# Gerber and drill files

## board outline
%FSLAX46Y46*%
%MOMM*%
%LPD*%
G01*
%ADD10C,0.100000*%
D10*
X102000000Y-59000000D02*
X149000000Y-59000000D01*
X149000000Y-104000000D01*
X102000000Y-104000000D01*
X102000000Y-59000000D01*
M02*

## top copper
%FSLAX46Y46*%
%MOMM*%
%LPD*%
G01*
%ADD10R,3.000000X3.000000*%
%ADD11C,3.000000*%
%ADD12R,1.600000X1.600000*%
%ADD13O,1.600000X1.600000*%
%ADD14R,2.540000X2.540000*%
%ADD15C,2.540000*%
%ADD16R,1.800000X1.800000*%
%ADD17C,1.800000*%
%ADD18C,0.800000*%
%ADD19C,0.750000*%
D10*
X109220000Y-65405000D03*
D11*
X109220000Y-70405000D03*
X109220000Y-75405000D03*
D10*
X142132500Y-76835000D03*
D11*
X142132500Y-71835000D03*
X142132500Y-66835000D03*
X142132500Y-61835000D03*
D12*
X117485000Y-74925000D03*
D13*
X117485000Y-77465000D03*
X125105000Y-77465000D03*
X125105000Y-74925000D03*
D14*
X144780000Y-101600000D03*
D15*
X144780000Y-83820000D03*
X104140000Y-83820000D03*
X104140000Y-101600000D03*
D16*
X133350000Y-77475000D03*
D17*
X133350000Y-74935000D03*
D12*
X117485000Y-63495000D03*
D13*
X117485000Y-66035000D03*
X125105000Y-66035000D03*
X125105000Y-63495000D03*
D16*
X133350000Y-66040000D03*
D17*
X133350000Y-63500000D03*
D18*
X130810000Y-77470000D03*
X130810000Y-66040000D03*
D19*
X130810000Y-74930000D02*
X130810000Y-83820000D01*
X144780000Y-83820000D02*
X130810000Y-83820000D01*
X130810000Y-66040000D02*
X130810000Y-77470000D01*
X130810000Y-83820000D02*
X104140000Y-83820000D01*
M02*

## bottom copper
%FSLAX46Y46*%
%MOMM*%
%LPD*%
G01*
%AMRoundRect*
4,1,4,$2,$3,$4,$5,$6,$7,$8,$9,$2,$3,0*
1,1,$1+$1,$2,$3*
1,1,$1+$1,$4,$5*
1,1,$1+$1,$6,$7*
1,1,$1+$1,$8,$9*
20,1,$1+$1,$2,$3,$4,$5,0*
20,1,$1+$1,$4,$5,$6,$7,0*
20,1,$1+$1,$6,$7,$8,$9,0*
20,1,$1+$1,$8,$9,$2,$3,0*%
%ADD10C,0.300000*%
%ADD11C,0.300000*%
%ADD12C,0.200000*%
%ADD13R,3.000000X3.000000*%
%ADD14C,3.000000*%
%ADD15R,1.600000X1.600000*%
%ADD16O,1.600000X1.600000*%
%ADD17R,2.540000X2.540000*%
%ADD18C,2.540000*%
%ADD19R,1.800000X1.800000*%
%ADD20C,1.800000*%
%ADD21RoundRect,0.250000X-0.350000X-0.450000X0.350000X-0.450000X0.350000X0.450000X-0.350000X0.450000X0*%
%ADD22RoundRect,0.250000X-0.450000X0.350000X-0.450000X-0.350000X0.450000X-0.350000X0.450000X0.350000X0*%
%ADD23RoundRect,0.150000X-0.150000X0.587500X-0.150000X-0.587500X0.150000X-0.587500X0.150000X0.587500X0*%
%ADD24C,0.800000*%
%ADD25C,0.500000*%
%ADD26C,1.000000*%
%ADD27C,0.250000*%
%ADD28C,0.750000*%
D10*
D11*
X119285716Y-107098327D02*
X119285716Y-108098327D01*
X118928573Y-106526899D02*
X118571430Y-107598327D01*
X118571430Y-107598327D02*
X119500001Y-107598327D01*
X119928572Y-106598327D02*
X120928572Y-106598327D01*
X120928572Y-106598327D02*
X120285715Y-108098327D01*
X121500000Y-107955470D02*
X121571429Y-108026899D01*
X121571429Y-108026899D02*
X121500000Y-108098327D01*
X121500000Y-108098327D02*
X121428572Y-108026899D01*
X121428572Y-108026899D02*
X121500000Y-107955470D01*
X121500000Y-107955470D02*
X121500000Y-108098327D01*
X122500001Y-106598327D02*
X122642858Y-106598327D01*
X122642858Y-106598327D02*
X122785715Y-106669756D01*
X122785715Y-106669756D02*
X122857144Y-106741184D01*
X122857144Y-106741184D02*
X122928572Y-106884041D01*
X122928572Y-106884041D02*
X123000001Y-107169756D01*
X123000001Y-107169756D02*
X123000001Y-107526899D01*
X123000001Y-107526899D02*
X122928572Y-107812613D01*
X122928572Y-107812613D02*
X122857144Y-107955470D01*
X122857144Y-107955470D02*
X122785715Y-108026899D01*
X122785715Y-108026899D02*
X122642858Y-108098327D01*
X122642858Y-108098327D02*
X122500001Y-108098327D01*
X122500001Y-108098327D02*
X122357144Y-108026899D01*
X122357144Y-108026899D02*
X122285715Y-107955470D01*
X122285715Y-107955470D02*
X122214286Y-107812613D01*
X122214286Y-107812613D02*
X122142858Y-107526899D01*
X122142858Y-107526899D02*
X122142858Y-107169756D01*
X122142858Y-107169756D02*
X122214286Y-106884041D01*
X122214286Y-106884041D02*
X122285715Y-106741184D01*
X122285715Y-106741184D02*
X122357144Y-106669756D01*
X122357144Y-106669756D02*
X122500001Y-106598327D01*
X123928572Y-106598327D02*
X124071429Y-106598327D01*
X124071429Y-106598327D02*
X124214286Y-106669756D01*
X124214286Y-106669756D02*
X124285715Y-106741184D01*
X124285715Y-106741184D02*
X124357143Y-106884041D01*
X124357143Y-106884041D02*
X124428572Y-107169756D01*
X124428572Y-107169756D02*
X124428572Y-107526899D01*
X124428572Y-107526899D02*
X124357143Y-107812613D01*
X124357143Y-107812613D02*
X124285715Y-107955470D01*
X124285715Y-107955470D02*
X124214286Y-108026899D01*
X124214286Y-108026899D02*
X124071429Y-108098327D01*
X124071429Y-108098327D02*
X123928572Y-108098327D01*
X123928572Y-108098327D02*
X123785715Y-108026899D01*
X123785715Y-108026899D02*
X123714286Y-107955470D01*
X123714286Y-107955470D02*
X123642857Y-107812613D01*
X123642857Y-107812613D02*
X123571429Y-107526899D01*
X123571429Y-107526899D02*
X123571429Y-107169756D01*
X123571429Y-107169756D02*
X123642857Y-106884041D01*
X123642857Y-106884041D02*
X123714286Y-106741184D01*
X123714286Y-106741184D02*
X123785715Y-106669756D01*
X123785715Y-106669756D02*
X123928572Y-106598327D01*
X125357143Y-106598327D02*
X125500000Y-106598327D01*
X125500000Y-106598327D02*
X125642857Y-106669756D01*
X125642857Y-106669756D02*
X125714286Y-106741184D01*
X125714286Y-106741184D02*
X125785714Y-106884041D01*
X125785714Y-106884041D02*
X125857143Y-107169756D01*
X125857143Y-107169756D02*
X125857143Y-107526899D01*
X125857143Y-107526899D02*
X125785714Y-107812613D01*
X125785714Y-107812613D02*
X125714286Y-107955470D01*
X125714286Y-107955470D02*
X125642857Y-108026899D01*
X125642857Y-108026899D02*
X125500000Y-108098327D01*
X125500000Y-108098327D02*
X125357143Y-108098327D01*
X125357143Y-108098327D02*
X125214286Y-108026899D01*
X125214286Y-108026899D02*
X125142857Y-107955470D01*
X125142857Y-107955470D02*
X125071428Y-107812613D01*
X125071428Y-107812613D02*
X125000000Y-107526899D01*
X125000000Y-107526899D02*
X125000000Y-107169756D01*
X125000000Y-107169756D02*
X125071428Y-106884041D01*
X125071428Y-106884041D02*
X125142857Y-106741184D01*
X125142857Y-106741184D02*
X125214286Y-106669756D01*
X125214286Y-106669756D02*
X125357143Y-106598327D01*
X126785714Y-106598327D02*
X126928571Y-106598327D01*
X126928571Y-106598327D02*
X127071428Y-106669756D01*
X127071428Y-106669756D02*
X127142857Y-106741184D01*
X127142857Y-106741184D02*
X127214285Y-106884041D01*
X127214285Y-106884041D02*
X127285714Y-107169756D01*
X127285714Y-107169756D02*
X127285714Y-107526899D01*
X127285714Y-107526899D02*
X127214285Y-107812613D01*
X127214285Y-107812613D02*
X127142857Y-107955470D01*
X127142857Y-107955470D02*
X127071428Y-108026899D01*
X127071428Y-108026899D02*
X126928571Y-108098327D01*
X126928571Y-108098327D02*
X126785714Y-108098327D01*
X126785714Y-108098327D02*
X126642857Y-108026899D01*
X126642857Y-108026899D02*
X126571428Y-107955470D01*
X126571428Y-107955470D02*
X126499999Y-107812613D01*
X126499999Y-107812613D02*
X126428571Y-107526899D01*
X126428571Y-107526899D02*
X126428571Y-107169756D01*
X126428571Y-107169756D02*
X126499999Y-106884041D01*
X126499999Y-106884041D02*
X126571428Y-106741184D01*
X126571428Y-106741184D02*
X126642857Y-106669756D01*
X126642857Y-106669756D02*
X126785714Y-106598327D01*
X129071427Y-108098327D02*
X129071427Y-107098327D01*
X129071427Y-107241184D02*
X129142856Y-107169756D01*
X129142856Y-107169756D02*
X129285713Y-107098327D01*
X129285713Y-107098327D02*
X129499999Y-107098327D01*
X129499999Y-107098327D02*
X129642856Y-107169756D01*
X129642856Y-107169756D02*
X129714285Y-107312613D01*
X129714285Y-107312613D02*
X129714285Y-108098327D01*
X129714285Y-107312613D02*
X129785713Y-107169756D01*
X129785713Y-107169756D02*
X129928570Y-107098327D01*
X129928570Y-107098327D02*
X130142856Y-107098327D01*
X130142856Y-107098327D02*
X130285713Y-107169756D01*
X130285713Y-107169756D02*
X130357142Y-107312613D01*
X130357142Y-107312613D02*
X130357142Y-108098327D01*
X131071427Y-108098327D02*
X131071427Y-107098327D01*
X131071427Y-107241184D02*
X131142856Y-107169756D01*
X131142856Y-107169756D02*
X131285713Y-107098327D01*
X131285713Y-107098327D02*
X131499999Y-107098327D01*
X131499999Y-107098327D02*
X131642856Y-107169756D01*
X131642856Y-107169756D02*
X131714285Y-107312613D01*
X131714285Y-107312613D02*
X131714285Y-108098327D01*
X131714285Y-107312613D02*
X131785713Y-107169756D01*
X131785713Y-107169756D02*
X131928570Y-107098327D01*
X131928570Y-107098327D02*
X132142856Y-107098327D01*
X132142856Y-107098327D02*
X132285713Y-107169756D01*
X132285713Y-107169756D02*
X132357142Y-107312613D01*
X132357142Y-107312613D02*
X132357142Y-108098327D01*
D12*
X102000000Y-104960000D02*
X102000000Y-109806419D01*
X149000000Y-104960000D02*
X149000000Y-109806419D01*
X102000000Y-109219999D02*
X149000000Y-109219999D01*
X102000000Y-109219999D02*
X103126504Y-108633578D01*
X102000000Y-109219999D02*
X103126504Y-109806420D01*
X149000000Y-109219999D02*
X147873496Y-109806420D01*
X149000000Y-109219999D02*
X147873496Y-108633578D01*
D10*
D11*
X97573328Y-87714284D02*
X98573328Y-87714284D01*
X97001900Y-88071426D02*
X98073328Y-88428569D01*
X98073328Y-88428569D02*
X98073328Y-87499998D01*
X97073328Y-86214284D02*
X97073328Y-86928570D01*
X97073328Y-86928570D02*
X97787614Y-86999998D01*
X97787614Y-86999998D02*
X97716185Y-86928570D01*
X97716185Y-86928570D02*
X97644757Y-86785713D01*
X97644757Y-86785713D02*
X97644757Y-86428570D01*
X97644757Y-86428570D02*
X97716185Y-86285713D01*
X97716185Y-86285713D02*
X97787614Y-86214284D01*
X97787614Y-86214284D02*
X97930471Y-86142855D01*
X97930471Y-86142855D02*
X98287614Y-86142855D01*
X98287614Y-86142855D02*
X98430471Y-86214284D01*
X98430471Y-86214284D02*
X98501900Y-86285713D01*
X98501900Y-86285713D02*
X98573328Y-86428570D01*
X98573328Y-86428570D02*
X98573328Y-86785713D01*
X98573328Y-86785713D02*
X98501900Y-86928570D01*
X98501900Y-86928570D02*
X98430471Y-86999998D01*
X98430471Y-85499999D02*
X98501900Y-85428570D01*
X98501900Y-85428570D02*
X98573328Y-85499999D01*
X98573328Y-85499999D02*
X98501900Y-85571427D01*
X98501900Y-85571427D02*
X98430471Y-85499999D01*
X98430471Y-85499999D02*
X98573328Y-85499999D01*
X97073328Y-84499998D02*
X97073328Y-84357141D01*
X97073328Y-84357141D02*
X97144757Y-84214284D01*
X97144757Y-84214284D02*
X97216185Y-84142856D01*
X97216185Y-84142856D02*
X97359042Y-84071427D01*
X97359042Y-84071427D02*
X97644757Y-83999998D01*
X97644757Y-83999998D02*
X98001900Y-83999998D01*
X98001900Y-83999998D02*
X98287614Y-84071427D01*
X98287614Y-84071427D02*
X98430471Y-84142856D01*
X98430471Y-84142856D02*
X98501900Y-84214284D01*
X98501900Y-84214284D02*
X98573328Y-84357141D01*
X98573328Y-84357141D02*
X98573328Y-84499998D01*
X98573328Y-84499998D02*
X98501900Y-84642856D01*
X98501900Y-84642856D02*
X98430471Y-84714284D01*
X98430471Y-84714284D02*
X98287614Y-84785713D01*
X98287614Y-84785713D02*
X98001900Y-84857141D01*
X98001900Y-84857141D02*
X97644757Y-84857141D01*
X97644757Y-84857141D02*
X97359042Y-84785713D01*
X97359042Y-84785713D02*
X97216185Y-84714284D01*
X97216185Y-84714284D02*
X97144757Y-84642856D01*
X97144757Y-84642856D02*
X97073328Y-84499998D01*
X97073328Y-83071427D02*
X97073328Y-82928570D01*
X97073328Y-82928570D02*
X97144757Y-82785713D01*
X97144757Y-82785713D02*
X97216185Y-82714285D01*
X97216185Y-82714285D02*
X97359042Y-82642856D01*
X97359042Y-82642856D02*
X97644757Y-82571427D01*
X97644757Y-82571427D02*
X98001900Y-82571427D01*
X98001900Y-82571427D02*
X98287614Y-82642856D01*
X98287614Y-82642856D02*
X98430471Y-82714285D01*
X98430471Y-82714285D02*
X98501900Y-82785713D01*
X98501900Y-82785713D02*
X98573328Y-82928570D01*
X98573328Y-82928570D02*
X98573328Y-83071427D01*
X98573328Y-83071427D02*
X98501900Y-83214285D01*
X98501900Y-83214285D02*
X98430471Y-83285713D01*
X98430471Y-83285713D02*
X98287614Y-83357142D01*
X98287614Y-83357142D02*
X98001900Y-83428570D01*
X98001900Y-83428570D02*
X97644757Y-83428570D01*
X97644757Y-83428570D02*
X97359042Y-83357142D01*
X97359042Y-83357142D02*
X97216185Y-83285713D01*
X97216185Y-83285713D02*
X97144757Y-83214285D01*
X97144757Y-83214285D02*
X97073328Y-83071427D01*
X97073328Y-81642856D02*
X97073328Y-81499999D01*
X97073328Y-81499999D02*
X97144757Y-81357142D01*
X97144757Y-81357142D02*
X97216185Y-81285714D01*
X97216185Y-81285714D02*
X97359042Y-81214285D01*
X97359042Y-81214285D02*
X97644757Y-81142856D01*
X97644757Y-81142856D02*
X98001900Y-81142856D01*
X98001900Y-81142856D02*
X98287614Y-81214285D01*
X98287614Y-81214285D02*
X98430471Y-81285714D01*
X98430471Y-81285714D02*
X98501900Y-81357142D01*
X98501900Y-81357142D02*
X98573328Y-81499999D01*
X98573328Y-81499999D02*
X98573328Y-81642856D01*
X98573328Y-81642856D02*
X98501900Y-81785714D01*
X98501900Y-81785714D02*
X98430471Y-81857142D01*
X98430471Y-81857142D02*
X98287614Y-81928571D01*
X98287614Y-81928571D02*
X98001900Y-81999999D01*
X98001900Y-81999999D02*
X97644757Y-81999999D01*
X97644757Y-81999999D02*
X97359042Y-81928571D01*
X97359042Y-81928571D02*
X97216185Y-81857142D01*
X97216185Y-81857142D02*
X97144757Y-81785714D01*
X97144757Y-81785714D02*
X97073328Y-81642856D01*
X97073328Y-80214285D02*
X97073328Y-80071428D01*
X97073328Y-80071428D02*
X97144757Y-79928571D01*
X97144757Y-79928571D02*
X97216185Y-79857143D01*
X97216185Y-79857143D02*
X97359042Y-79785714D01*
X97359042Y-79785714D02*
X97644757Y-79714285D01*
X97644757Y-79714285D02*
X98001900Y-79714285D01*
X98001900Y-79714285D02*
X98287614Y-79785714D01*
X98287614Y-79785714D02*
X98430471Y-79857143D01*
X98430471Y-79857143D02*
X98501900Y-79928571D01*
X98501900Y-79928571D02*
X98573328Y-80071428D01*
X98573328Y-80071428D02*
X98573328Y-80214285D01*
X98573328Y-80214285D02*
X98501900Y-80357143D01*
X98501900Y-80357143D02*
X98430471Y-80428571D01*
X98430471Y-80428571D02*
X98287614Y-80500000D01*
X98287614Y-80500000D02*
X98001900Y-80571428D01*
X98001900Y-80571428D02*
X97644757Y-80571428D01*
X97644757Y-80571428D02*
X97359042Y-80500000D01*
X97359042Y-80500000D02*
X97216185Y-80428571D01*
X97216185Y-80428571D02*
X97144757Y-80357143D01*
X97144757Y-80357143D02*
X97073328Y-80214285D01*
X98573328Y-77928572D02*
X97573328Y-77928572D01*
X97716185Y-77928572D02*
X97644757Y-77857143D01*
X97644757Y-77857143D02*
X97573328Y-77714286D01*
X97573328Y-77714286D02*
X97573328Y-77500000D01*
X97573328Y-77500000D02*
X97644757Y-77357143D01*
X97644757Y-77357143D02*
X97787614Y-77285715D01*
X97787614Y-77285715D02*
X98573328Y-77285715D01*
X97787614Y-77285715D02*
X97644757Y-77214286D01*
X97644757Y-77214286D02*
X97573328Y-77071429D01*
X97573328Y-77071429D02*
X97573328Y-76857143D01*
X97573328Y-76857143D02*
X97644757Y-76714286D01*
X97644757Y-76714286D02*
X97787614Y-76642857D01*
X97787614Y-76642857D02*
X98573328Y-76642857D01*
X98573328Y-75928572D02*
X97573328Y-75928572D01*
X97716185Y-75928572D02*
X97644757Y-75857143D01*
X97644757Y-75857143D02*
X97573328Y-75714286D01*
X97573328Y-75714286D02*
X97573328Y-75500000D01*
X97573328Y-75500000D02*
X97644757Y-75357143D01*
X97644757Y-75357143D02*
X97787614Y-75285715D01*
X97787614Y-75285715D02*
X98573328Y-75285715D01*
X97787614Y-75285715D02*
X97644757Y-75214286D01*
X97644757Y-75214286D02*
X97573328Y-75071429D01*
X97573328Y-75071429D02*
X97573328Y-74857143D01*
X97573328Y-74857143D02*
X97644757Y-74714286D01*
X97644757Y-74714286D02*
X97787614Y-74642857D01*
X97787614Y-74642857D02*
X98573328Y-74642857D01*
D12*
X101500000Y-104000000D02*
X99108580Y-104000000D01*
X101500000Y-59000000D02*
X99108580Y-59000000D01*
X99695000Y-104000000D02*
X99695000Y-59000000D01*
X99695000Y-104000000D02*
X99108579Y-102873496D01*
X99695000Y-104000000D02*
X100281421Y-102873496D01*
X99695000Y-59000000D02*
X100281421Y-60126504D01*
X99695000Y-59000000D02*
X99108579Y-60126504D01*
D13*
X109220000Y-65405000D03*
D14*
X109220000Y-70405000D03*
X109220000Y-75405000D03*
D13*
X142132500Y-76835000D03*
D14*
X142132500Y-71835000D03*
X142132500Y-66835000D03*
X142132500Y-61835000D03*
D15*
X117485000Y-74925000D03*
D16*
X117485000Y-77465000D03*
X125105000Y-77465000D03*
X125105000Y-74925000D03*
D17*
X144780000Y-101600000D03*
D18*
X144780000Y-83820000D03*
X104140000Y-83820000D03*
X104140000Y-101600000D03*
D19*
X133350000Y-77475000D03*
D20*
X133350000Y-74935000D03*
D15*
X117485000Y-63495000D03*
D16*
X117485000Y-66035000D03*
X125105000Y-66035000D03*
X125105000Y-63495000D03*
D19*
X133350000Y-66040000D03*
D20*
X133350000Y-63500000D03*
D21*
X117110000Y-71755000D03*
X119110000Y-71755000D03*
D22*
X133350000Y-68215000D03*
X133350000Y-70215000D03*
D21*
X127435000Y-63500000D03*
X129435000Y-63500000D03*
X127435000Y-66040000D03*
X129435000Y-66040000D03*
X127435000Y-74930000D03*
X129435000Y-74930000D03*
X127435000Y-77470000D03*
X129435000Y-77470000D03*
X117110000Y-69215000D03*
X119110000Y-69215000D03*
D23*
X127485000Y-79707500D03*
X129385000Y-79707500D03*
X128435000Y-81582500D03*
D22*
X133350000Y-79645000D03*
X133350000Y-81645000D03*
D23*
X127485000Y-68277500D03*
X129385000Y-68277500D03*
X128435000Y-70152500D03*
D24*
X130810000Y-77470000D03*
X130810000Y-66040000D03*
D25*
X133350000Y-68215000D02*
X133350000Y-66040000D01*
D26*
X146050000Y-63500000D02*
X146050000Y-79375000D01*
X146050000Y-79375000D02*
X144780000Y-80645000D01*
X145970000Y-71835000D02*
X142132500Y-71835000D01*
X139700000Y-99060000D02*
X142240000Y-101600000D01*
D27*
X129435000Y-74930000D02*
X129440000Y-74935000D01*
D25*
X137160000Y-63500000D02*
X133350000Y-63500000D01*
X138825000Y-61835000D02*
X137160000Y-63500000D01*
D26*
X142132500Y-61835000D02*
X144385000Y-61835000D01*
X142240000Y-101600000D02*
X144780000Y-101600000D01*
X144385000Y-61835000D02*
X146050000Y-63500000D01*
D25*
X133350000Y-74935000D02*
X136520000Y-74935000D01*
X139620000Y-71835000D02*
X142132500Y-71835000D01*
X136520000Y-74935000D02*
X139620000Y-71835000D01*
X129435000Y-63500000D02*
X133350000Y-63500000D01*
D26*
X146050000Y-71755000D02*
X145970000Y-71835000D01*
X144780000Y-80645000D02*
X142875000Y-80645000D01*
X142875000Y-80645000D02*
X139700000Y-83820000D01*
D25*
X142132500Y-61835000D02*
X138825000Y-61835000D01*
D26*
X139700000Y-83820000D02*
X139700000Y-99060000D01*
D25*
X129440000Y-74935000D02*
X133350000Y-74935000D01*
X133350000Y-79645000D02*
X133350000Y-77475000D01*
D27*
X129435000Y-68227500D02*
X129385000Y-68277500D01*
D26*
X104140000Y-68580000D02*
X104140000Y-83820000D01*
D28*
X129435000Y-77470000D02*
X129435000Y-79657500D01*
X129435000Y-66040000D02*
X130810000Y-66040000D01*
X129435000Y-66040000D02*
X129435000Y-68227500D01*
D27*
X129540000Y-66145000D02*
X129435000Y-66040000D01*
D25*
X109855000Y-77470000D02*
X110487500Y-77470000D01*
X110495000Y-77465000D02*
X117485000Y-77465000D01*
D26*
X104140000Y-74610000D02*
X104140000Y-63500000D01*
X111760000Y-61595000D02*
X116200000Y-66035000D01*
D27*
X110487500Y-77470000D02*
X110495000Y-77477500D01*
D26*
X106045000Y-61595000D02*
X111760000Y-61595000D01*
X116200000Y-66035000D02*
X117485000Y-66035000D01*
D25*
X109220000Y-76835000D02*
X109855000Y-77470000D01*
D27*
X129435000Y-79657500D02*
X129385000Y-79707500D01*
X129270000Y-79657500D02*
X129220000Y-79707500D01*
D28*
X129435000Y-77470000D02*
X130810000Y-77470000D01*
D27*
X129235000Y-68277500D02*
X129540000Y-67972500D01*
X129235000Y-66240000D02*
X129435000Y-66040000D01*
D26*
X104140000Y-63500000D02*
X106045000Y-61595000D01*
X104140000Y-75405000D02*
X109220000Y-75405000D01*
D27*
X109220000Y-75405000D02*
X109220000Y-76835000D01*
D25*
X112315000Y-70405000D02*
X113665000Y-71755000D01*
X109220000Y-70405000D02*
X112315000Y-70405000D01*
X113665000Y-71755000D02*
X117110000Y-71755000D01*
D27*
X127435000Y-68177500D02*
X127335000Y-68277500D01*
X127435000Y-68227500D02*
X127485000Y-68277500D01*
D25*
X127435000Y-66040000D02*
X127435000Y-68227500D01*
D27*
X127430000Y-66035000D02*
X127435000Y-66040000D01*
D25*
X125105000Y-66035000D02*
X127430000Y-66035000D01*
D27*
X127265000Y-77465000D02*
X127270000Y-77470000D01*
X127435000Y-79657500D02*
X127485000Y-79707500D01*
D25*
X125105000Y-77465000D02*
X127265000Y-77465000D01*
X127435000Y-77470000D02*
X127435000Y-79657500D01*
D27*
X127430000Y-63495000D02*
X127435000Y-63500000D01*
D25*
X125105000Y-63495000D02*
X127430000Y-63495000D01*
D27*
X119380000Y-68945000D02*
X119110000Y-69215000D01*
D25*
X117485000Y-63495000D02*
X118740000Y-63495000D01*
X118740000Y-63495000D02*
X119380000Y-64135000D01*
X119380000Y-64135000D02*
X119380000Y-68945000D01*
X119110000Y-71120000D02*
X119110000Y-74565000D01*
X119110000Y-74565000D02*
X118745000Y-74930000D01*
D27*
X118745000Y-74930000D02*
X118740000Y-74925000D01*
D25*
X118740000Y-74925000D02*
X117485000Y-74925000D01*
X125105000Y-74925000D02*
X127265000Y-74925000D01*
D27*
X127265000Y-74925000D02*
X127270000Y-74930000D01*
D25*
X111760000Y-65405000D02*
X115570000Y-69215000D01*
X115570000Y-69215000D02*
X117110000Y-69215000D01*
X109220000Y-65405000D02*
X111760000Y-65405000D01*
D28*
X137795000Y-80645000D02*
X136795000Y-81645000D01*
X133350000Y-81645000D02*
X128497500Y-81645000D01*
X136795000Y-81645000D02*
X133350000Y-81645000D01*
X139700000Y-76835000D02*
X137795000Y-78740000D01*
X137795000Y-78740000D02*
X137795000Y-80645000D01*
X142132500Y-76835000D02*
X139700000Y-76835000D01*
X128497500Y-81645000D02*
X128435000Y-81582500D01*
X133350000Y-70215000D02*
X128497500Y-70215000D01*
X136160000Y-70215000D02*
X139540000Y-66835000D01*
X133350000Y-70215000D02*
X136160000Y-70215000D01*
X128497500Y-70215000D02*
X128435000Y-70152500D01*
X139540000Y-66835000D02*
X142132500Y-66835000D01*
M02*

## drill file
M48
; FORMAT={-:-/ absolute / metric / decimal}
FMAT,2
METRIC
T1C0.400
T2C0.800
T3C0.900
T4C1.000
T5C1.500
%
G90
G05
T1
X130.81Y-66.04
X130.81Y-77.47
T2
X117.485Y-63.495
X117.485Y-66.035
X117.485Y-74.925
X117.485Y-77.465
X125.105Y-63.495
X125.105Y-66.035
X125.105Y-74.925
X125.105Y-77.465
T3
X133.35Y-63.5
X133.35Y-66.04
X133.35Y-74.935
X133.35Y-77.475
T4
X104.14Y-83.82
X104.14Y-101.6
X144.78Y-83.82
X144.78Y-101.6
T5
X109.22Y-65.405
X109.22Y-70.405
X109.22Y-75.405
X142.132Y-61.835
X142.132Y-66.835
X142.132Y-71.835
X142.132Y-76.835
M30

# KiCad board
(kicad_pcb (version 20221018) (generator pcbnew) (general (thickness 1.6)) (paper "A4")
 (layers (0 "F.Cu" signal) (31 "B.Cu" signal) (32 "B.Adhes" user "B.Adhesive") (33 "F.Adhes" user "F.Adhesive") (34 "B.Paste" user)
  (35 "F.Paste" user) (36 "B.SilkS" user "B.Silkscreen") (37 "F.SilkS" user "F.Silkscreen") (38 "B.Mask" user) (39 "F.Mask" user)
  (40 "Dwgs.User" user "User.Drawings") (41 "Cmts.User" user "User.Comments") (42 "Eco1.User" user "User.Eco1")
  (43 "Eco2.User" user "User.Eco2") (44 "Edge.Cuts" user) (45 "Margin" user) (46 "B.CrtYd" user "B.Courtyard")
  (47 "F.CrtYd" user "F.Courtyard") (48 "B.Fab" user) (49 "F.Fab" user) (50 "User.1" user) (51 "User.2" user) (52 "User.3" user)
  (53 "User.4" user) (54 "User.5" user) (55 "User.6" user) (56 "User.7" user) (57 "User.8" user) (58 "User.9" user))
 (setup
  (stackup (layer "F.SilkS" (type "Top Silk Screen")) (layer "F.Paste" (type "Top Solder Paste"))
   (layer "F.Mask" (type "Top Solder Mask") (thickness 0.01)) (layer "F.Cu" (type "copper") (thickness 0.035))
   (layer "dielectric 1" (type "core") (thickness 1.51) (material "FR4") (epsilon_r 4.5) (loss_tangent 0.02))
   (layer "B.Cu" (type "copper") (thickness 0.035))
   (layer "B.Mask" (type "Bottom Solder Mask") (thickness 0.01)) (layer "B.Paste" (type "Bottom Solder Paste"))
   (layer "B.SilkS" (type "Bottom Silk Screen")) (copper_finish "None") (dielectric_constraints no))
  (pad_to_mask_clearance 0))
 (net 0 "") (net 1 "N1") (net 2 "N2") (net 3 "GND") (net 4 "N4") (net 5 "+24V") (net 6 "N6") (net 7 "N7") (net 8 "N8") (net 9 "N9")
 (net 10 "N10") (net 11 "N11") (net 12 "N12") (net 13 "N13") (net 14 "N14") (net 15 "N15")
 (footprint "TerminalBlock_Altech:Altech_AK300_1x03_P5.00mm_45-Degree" (layer "F.Cu") (at 109.22 65.405 -90)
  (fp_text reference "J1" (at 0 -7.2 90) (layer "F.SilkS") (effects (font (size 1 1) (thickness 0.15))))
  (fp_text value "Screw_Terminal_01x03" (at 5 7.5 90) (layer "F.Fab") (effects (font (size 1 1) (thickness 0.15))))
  (pad "1" thru_hole rect (at 0 0 270) (size 3 3) (drill 1.5) (layers "*.Cu" "*.Mask") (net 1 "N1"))
  (pad "2" thru_hole circle (at 5 0 270) (size 3 3) (drill 1.5) (layers "*.Cu" "*.Mask") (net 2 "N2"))
  (pad "3" thru_hole circle (at 10 0 270) (size 3 3) (drill 1.5) (layers "*.Cu" "*.Mask") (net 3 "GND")))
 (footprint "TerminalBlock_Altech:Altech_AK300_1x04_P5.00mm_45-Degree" (layer "F.Cu") (at 142.1325 76.835 90)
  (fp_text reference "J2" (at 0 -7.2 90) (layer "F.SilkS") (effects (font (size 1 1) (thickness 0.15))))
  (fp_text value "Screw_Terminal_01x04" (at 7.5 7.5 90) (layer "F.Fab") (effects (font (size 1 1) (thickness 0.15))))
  (pad "1" thru_hole rect (at 0 0 90) (size 3 3) (drill 1.5) (layers "*.Cu" "*.Mask") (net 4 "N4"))
  (pad "2" thru_hole circle (at 5 0 90) (size 3 3) (drill 1.5) (layers "*.Cu" "*.Mask") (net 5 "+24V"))
  (pad "3" thru_hole circle (at 10 0 90) (size 3 3) (drill 1.5) (layers "*.Cu" "*.Mask") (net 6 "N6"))
  (pad "4" thru_hole circle (at 15 0 90) (size 3 3) (drill 1.5) (layers "*.Cu" "*.Mask") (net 5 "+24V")))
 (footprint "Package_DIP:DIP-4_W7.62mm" (layer "F.Cu") (at 117.485 74.925)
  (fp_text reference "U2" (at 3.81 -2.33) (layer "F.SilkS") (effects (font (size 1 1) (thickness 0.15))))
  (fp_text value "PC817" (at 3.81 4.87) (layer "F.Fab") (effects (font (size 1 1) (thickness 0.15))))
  (pad "1" thru_hole rect (at 0 0) (size 1.6 1.6) (drill 0.8) (layers "*.Cu" "*.Mask") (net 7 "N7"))
  (pad "2" thru_hole oval (at 0 2.54) (size 1.6 1.6) (drill 0.8) (layers "*.Cu" "*.Mask") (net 3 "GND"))
  (pad "3" thru_hole oval (at 7.62 2.54) (size 1.6 1.6) (drill 0.8) (layers "*.Cu" "*.Mask") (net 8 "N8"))
  (pad "4" thru_hole oval (at 7.62 0) (size 1.6 1.6) (drill 0.8) (layers "*.Cu" "*.Mask") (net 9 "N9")))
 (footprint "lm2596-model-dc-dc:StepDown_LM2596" (layer "F.Cu") (at 144.78 101.6 180)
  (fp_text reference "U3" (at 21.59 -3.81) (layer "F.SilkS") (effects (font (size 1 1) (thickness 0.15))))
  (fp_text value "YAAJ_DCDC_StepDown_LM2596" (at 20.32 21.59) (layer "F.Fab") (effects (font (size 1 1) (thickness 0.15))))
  (pad "1" thru_hole rect (at 0 0 180) (size 2.54 2.54) (drill 1) (layers "*.Cu" "*.Mask") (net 5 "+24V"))
  (pad "2" thru_hole circle (at 0 17.78 180) (size 2.54 2.54) (drill 1) (layers "*.Cu" "*.Mask") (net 3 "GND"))
  (pad "3" thru_hole circle (at 40.64 17.78 180) (size 2.54 2.54) (drill 1) (layers "*.Cu" "*.Mask") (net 3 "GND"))
  (pad "4" thru_hole circle (at 40.64 0 180) (size 2.54 2.54) (drill 1) (layers "*.Cu" "*.Mask") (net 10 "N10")))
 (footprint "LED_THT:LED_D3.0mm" (layer "F.Cu") (at 133.35 77.475 90)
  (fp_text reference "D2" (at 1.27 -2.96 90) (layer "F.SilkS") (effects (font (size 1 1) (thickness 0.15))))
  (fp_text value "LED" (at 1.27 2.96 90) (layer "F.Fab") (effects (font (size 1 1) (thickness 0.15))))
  (pad "1" thru_hole rect (at 0 0 90) (size 1.8 1.8) (drill 0.9) (layers "*.Cu" "*.Mask") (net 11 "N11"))
  (pad "2" thru_hole circle (at 2.54 0 90) (size 1.8 1.8) (drill 0.9) (layers "*.Cu" "*.Mask") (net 5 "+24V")))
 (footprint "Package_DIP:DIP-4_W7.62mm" (layer "F.Cu") (at 117.485 63.495)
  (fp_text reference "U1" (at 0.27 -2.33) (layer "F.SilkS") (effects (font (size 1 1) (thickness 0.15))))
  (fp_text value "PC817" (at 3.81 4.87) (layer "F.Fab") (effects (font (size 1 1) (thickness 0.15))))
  (pad "1" thru_hole rect (at 0 0) (size 1.6 1.6) (drill 0.8) (layers "*.Cu" "*.Mask") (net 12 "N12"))
  (pad "2" thru_hole oval (at 0 2.54) (size 1.6 1.6) (drill 0.8) (layers "*.Cu" "*.Mask") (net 3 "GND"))
  (pad "3" thru_hole oval (at 7.62 2.54) (size 1.6 1.6) (drill 0.8) (layers "*.Cu" "*.Mask") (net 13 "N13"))
  (pad "4" thru_hole oval (at 7.62 0) (size 1.6 1.6) (drill 0.8) (layers "*.Cu" "*.Mask") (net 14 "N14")))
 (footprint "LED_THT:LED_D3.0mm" (layer "F.Cu") (at 133.35 66.04 90)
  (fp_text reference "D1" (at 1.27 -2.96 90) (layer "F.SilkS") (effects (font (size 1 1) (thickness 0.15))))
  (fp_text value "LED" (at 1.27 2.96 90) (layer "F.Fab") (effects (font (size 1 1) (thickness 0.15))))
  (pad "1" thru_hole rect (at 0 0 90) (size 1.8 1.8) (drill 0.9) (layers "*.Cu" "*.Mask") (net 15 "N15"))
  (pad "2" thru_hole circle (at 2.54 0 90) (size 1.8 1.8) (drill 0.9) (layers "*.Cu" "*.Mask") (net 5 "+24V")))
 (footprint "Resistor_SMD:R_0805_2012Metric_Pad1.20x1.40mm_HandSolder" (layer "B.Cu") (at 118.11 71.755)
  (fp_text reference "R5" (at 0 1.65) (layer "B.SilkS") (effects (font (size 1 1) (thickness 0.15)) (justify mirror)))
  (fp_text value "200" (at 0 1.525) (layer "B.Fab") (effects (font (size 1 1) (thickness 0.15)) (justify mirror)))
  (pad "1" smd roundrect (at -1 0) (size 1.2 1.4) (layers "B.Cu" "B.Paste" "B.Mask") (roundrect_rratio 0.208333) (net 2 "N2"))
  (pad "2" smd roundrect (at 1 0) (size 1.2 1.4) (layers "B.Cu" "B.Paste" "B.Mask") (roundrect_rratio 0.208333) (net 7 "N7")))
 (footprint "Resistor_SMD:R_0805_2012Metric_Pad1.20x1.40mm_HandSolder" (layer "B.Cu") (at 133.35 69.215 -90)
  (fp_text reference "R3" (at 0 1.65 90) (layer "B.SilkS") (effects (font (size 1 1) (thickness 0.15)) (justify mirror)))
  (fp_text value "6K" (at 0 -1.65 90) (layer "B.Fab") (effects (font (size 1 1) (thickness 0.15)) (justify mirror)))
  (pad "1" smd roundrect (at -1 0 270) (size 1.2 1.4) (layers "B.Cu" "B.Paste" "B.Mask") (roundrect_rratio 0.208333) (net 15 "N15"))
  (pad "2" smd roundrect (at 1 0 270) (size 1.2 1.4) (layers "B.Cu" "B.Paste" "B.Mask") (roundrect_rratio 0.208333) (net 6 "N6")))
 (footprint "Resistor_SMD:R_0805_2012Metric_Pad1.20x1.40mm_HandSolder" (layer "B.Cu") (at 128.435 63.5)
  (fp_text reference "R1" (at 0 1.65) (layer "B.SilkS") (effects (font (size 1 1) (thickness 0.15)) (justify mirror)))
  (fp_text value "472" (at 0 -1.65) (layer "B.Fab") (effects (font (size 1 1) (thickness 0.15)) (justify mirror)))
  (pad "1" smd roundrect (at -1 0) (size 1.2 1.4) (layers "B.Cu" "B.Paste" "B.Mask") (roundrect_rratio 0.208333) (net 14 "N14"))
  (pad "2" smd roundrect (at 1 0) (size 1.2 1.4) (layers "B.Cu" "B.Paste" "B.Mask") (roundrect_rratio 0.208333) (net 5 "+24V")))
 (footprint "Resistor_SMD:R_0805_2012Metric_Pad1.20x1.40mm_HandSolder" (layer "B.Cu") (at 128.435 66.04)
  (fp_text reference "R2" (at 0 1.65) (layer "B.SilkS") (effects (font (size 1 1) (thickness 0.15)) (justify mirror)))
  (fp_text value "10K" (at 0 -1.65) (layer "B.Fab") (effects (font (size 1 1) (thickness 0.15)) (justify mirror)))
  (pad "1" smd roundrect (at -1 0) (size 1.2 1.4) (layers "B.Cu" "B.Paste" "B.Mask") (roundrect_rratio 0.208333) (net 13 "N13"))
  (pad "2" smd roundrect (at 1 0) (size 1.2 1.4) (layers "B.Cu" "B.Paste" "B.Mask") (roundrect_rratio 0.208333) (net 3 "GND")))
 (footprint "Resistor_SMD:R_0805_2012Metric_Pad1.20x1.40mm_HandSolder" (layer "B.Cu") (at 128.435 74.93)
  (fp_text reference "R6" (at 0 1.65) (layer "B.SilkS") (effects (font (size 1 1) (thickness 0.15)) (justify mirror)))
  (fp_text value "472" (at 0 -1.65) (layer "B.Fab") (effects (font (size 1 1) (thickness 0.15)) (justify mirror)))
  (pad "1" smd roundrect (at -1 0) (size 1.2 1.4) (layers "B.Cu" "B.Paste" "B.Mask") (roundrect_rratio 0.208333) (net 9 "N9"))
  (pad "2" smd roundrect (at 1 0) (size 1.2 1.4) (layers "B.Cu" "B.Paste" "B.Mask") (roundrect_rratio 0.208333) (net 5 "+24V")))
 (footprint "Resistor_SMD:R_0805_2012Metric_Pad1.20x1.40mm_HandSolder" (layer "B.Cu") (at 128.435 77.47)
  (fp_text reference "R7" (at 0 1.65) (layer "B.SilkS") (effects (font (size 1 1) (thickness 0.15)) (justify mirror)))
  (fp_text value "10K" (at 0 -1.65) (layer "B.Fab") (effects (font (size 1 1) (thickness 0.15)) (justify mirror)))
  (pad "1" smd roundrect (at -1 0) (size 1.2 1.4) (layers "B.Cu" "B.Paste" "B.Mask") (roundrect_rratio 0.208333) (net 8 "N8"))
  (pad "2" smd roundrect (at 1 0) (size 1.2 1.4) (layers "B.Cu" "B.Paste" "B.Mask") (roundrect_rratio 0.208333) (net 3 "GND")))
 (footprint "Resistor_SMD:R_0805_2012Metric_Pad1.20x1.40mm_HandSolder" (layer "B.Cu") (at 118.11 69.215)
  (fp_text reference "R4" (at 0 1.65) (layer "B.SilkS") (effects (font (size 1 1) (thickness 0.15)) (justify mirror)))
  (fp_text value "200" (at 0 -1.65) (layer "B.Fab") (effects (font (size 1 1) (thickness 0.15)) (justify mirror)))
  (pad "1" smd roundrect (at -1 0) (size 1.2 1.4) (layers "B.Cu" "B.Paste" "B.Mask") (roundrect_rratio 0.208333) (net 1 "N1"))
  (pad "2" smd roundrect (at 1 0) (size 1.2 1.4) (layers "B.Cu" "B.Paste" "B.Mask") (roundrect_rratio 0.208333) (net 12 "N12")))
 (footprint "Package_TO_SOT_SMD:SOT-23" (layer "B.Cu") (at 128.435 80.645 -90)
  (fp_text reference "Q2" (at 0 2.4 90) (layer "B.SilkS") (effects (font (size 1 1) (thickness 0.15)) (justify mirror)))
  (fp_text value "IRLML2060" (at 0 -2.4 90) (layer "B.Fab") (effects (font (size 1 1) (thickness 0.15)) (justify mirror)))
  (pad "1" smd roundrect (at -0.9375 0.95 270) (size 1.475 0.6) (layers "B.Cu" "B.Paste" "B.Mask") (roundrect_rratio 0.25) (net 8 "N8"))
  (pad "2" smd roundrect (at -0.9375 -0.95 270) (size 1.475 0.6) (layers "B.Cu" "B.Paste" "B.Mask") (roundrect_rratio 0.25) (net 3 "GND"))
  (pad "3" smd roundrect (at 0.9375 0 270) (size 1.475 0.6) (layers "B.Cu" "B.Paste" "B.Mask") (roundrect_rratio 0.25) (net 4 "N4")))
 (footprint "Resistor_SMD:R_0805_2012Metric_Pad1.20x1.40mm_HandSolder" (layer "B.Cu") (at 133.35 80.645 -90)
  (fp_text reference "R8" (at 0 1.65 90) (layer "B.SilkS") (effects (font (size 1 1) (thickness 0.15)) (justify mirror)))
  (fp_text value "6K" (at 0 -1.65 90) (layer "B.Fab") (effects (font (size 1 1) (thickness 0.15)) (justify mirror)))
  (pad "1" smd roundrect (at -1 0 270) (size 1.2 1.4) (layers "B.Cu" "B.Paste" "B.Mask") (roundrect_rratio 0.208333) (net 11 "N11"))
  (pad "2" smd roundrect (at 1 0 270) (size 1.2 1.4) (layers "B.Cu" "B.Paste" "B.Mask") (roundrect_rratio 0.208333) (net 4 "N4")))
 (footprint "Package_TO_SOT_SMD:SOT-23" (layer "B.Cu") (at 128.435 69.215 -90)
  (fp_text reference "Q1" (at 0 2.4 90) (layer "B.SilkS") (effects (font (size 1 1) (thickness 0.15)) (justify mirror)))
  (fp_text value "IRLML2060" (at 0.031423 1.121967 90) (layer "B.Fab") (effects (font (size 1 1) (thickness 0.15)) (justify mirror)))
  (pad "1" smd roundrect (at -0.9375 0.95 270) (size 1.475 0.6) (layers "B.Cu" "B.Paste" "B.Mask") (roundrect_rratio 0.25) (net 13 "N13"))
  (pad "2" smd roundrect (at -0.9375 -0.95 270) (size 1.475 0.6) (layers "B.Cu" "B.Paste" "B.Mask") (roundrect_rratio 0.25) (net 3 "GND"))
  (pad "3" smd roundrect (at 0.9375 0 270) (size 1.475 0.6) (layers "B.Cu" "B.Paste" "B.Mask") (roundrect_rratio 0.25) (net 6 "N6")))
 (gr_rect (start 102 59) (end 149 104) (stroke (width 0.1) (type default)) (fill none) (layer "Edge.Cuts"))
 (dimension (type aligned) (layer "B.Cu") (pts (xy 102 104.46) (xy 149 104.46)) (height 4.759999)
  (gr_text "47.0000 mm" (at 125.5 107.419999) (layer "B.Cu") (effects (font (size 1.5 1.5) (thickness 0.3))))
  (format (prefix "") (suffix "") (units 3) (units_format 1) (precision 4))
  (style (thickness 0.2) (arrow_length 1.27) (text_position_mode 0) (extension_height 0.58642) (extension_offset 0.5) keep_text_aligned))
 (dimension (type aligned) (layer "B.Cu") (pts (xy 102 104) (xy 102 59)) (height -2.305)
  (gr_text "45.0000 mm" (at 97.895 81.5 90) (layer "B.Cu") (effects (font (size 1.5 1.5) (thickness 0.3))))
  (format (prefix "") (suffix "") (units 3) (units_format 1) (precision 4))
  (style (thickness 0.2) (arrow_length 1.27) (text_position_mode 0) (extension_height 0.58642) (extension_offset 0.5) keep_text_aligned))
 (segment (start 133.35 68.215) (end 133.35 66.04) (width 0.5) (layer "B.Cu") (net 15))
 (segment (start 146.05 63.5) (end 146.05 79.375) (width 1) (layer "B.Cu") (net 5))
 (segment (start 146.05 79.375) (end 144.78 80.645) (width 1) (layer "B.Cu") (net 5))
 (segment (start 145.97 71.835) (end 142.1325 71.835) (width 1) (layer "B.Cu") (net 5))
 (segment (start 139.7 99.06) (end 142.24 101.6) (width 1) (layer "B.Cu") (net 5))
 (segment (start 129.435 74.93) (end 129.44 74.935) (width 0.25) (layer "B.Cu") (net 5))
 (segment (start 137.16 63.5) (end 133.35 63.5) (width 0.5) (layer "B.Cu") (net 5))
 (segment (start 138.825 61.835) (end 137.16 63.5) (width 0.5) (layer "B.Cu") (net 5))
 (segment (start 142.1325 61.835) (end 144.385 61.835) (width 1) (layer "B.Cu") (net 5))
 (segment (start 142.24 101.6) (end 144.78 101.6) (width 1) (layer "B.Cu") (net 5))
 (segment (start 144.385 61.835) (end 146.05 63.5) (width 1) (layer "B.Cu") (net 5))
 (segment (start 133.35 74.935) (end 136.52 74.935) (width 0.5) (layer "B.Cu") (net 5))
 (segment (start 139.62 71.835) (end 142.1325 71.835) (width 0.5) (layer "B.Cu") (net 5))
 (segment (start 136.52 74.935) (end 139.62 71.835) (width 0.5) (layer "B.Cu") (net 5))
 (segment (start 129.435 63.5) (end 133.35 63.5) (width 0.5) (layer "B.Cu") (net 5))
 (segment (start 146.05 71.755) (end 145.97 71.835) (width 1) (layer "B.Cu") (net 5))
 (segment (start 144.78 80.645) (end 142.875 80.645) (width 1) (layer "B.Cu") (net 5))
 (segment (start 142.875 80.645) (end 139.7 83.82) (width 1) (layer "B.Cu") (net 5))
 (segment (start 142.1325 61.835) (end 138.825 61.835) (width 0.5) (layer "B.Cu") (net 5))
 (segment (start 139.7 83.82) (end 139.7 99.06) (width 1) (layer "B.Cu") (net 5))
 (segment (start 129.44 74.935) (end 133.35 74.935) (width 0.5) (layer "B.Cu") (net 5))
 (segment (start 133.35 79.645) (end 133.35 77.475) (width 0.5) (layer "B.Cu") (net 11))
 (segment (start 130.81 74.93) (end 130.81 83.82) (width 0.75) (layer "F.Cu") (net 3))
 (segment (start 144.78 83.82) (end 130.81 83.82) (width 0.75) (layer "F.Cu") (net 3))
 (segment (start 130.81 66.04) (end 130.81 77.47) (width 0.75) (layer "F.Cu") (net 3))
 (segment (start 130.81 83.82) (end 104.14 83.82) (width 0.75) (layer "F.Cu") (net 3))
 (via (at 130.81 77.47) (size 0.8) (drill 0.4) (layers "F.Cu" "B.Cu") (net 3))
 (via (at 130.81 66.04) (size 0.8) (drill 0.4) (layers "F.Cu" "B.Cu") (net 3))
 (segment (start 129.435 68.2275) (end 129.385 68.2775) (width 0.25) (layer "B.Cu") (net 3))
 (segment (start 104.14 68.58) (end 104.14 83.82) (width 1) (layer "B.Cu") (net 3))
 (segment (start 129.435 77.47) (end 129.435 79.6575) (width 0.75) (layer "B.Cu") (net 3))
 (segment (start 129.435 66.04) (end 130.81 66.04) (width 0.75) (layer "B.Cu") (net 3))
 (segment (start 129.435 66.04) (end 129.435 68.2275) (width 0.75) (layer "B.Cu") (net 3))
 (segment (start 129.54 66.145) (end 129.435 66.04) (width 0.25) (layer "B.Cu") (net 3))
 (segment (start 109.855 77.47) (end 110.4875 77.47) (width 0.5) (layer "B.Cu") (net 3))
 (segment (start 110.495 77.465) (end 117.485 77.465) (width 0.5) (layer "B.Cu") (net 3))
 (segment (start 104.14 74.61) (end 104.14 63.5) (width 1) (layer "B.Cu") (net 3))
 (segment (start 111.76 61.595) (end 116.2 66.035) (width 1) (layer "B.Cu") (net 3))
 (segment (start 110.4875 77.47) (end 110.495 77.4775) (width 0.25) (layer "B.Cu") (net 3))
 (segment (start 106.045 61.595) (end 111.76 61.595) (width 1) (layer "B.Cu") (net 3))
 (segment (start 116.2 66.035) (end 117.485 66.035) (width 1) (layer "B.Cu") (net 3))
 (segment (start 109.22 76.835) (end 109.855 77.47) (width 0.5) (layer "B.Cu") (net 3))
 (segment (start 129.435 79.6575) (end 129.385 79.7075) (width 0.25) (layer "B.Cu") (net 3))
 (segment (start 129.27 79.6575) (end 129.22 79.7075) (width 0.25) (layer "B.Cu") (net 3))
 (segment (start 129.435 77.47) (end 130.81 77.47) (width 0.75) (layer "B.Cu") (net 3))
 (segment (start 129.235 68.2775) (end 129.54 67.9725) (width 0.25) (layer "B.Cu") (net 3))
 (segment (start 129.235 66.24) (end 129.435 66.04) (width 0.25) (layer "B.Cu") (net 3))
 (segment (start 104.14 63.5) (end 106.045 61.595) (width 1) (layer "B.Cu") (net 3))
 (segment (start 104.14 75.405) (end 109.22 75.405) (width 1) (layer "B.Cu") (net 3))
 (segment (start 109.22 75.405) (end 109.22 76.835) (width 0.25) (layer "B.Cu") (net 3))
 (segment (start 112.315 70.405) (end 113.665 71.755) (width 0.5) (layer "B.Cu") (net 2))
 (segment (start 109.22 70.405) (end 112.315 70.405) (width 0.5) (layer "B.Cu") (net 2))
 (segment (start 113.665 71.755) (end 117.11 71.755) (width 0.5) (layer "B.Cu") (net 2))
 (segment (start 127.435 68.1775) (end 127.335 68.2775) (width 0.25) (layer "B.Cu") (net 13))
 (segment (start 127.435 68.2275) (end 127.485 68.2775) (width 0.25) (layer "B.Cu") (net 13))
 (segment (start 127.435 66.04) (end 127.435 68.2275) (width 0.5) (layer "B.Cu") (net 13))
 (segment (start 127.43 66.035) (end 127.435 66.04) (width 0.25) (layer "B.Cu") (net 13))
 (segment (start 125.105 66.035) (end 127.43 66.035) (width 0.5) (layer "B.Cu") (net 13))
 (segment (start 127.265 77.465) (end 127.27 77.47) (width 0.25) (layer "B.Cu") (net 8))
 (segment (start 127.435 79.6575) (end 127.485 79.7075) (width 0.25) (layer "B.Cu") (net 8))
 (segment (start 125.105 77.465) (end 127.265 77.465) (width 0.5) (layer "B.Cu") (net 8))
 (segment (start 127.435 77.47) (end 127.435 79.6575) (width 0.5) (layer "B.Cu") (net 8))
 (segment (start 127.43 63.495) (end 127.435 63.5) (width 0.25) (layer "B.Cu") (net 14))
 (segment (start 125.105 63.495) (end 127.43 63.495) (width 0.5) (layer "B.Cu") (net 14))
 (segment (start 119.38 68.945) (end 119.11 69.215) (width 0.25) (layer "B.Cu") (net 12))
 (segment (start 117.485 63.495) (end 118.74 63.495) (width 0.5) (layer "B.Cu") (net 12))
 (segment (start 118.74 63.495) (end 119.38 64.135) (width 0.5) (layer "B.Cu") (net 12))
 (segment (start 119.38 64.135) (end 119.38 68.945) (width 0.5) (layer "B.Cu") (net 12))
 (segment (start 119.11 71.12) (end 119.11 74.565) (width 0.5) (layer "B.Cu") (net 7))
 (segment (start 119.11 74.565) (end 118.745 74.93) (width 0.5) (layer "B.Cu") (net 7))
 (segment (start 118.745 74.93) (end 118.74 74.925) (width 0.25) (layer "B.Cu") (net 7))
 (segment (start 118.74 74.925) (end 117.485 74.925) (width 0.5) (layer "B.Cu") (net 7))
 (segment (start 125.105 74.925) (end 127.265 74.925) (width 0.5) (layer "B.Cu") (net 9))
 (segment (start 127.265 74.925) (end 127.27 74.93) (width 0.25) (layer "B.Cu") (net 9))
 (segment (start 111.76 65.405) (end 115.57 69.215) (width 0.5) (layer "B.Cu") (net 1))
 (segment (start 115.57 69.215) (end 117.11 69.215) (width 0.5) (layer "B.Cu") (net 1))
 (segment (start 109.22 65.405) (end 111.76 65.405) (width 0.5) (layer "B.Cu") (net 1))
 (segment (start 137.795 80.645) (end 136.795 81.645) (width 0.75) (layer "B.Cu") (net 4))
 (segment (start 133.35 81.645) (end 128.4975 81.645) (width 0.75) (layer "B.Cu") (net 4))
 (segment (start 136.795 81.645) (end 133.35 81.645) (width 0.75) (layer "B.Cu") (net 4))
 (segment (start 139.7 76.835) (end 137.795 78.74) (width 0.75) (layer "B.Cu") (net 4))
 (segment (start 137.795 78.74) (end 137.795 80.645) (width 0.75) (layer "B.Cu") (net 4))
 (segment (start 142.1325 76.835) (end 139.7 76.835) (width 0.75) (layer "B.Cu") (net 4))
 (segment (start 128.4975 81.645) (end 128.435 81.5825) (width 0.75) (layer "B.Cu") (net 4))
 (segment (start 133.35 70.215) (end 128.4975 70.215) (width 0.75) (layer "B.Cu") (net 6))
 (segment (start 136.16 70.215) (end 139.54 66.835) (width 0.75) (layer "B.Cu") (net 6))
 (segment (start 133.35 70.215) (end 136.16 70.215) (width 0.75) (layer "B.Cu") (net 6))
 (segment (start 128.4975 70.215) (end 128.435 70.1525) (width 0.75) (layer "B.Cu") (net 6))
 (segment (start 139.54 66.835) (end 142.1325 66.835) (width 0.75) (layer "B.Cu") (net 6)))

